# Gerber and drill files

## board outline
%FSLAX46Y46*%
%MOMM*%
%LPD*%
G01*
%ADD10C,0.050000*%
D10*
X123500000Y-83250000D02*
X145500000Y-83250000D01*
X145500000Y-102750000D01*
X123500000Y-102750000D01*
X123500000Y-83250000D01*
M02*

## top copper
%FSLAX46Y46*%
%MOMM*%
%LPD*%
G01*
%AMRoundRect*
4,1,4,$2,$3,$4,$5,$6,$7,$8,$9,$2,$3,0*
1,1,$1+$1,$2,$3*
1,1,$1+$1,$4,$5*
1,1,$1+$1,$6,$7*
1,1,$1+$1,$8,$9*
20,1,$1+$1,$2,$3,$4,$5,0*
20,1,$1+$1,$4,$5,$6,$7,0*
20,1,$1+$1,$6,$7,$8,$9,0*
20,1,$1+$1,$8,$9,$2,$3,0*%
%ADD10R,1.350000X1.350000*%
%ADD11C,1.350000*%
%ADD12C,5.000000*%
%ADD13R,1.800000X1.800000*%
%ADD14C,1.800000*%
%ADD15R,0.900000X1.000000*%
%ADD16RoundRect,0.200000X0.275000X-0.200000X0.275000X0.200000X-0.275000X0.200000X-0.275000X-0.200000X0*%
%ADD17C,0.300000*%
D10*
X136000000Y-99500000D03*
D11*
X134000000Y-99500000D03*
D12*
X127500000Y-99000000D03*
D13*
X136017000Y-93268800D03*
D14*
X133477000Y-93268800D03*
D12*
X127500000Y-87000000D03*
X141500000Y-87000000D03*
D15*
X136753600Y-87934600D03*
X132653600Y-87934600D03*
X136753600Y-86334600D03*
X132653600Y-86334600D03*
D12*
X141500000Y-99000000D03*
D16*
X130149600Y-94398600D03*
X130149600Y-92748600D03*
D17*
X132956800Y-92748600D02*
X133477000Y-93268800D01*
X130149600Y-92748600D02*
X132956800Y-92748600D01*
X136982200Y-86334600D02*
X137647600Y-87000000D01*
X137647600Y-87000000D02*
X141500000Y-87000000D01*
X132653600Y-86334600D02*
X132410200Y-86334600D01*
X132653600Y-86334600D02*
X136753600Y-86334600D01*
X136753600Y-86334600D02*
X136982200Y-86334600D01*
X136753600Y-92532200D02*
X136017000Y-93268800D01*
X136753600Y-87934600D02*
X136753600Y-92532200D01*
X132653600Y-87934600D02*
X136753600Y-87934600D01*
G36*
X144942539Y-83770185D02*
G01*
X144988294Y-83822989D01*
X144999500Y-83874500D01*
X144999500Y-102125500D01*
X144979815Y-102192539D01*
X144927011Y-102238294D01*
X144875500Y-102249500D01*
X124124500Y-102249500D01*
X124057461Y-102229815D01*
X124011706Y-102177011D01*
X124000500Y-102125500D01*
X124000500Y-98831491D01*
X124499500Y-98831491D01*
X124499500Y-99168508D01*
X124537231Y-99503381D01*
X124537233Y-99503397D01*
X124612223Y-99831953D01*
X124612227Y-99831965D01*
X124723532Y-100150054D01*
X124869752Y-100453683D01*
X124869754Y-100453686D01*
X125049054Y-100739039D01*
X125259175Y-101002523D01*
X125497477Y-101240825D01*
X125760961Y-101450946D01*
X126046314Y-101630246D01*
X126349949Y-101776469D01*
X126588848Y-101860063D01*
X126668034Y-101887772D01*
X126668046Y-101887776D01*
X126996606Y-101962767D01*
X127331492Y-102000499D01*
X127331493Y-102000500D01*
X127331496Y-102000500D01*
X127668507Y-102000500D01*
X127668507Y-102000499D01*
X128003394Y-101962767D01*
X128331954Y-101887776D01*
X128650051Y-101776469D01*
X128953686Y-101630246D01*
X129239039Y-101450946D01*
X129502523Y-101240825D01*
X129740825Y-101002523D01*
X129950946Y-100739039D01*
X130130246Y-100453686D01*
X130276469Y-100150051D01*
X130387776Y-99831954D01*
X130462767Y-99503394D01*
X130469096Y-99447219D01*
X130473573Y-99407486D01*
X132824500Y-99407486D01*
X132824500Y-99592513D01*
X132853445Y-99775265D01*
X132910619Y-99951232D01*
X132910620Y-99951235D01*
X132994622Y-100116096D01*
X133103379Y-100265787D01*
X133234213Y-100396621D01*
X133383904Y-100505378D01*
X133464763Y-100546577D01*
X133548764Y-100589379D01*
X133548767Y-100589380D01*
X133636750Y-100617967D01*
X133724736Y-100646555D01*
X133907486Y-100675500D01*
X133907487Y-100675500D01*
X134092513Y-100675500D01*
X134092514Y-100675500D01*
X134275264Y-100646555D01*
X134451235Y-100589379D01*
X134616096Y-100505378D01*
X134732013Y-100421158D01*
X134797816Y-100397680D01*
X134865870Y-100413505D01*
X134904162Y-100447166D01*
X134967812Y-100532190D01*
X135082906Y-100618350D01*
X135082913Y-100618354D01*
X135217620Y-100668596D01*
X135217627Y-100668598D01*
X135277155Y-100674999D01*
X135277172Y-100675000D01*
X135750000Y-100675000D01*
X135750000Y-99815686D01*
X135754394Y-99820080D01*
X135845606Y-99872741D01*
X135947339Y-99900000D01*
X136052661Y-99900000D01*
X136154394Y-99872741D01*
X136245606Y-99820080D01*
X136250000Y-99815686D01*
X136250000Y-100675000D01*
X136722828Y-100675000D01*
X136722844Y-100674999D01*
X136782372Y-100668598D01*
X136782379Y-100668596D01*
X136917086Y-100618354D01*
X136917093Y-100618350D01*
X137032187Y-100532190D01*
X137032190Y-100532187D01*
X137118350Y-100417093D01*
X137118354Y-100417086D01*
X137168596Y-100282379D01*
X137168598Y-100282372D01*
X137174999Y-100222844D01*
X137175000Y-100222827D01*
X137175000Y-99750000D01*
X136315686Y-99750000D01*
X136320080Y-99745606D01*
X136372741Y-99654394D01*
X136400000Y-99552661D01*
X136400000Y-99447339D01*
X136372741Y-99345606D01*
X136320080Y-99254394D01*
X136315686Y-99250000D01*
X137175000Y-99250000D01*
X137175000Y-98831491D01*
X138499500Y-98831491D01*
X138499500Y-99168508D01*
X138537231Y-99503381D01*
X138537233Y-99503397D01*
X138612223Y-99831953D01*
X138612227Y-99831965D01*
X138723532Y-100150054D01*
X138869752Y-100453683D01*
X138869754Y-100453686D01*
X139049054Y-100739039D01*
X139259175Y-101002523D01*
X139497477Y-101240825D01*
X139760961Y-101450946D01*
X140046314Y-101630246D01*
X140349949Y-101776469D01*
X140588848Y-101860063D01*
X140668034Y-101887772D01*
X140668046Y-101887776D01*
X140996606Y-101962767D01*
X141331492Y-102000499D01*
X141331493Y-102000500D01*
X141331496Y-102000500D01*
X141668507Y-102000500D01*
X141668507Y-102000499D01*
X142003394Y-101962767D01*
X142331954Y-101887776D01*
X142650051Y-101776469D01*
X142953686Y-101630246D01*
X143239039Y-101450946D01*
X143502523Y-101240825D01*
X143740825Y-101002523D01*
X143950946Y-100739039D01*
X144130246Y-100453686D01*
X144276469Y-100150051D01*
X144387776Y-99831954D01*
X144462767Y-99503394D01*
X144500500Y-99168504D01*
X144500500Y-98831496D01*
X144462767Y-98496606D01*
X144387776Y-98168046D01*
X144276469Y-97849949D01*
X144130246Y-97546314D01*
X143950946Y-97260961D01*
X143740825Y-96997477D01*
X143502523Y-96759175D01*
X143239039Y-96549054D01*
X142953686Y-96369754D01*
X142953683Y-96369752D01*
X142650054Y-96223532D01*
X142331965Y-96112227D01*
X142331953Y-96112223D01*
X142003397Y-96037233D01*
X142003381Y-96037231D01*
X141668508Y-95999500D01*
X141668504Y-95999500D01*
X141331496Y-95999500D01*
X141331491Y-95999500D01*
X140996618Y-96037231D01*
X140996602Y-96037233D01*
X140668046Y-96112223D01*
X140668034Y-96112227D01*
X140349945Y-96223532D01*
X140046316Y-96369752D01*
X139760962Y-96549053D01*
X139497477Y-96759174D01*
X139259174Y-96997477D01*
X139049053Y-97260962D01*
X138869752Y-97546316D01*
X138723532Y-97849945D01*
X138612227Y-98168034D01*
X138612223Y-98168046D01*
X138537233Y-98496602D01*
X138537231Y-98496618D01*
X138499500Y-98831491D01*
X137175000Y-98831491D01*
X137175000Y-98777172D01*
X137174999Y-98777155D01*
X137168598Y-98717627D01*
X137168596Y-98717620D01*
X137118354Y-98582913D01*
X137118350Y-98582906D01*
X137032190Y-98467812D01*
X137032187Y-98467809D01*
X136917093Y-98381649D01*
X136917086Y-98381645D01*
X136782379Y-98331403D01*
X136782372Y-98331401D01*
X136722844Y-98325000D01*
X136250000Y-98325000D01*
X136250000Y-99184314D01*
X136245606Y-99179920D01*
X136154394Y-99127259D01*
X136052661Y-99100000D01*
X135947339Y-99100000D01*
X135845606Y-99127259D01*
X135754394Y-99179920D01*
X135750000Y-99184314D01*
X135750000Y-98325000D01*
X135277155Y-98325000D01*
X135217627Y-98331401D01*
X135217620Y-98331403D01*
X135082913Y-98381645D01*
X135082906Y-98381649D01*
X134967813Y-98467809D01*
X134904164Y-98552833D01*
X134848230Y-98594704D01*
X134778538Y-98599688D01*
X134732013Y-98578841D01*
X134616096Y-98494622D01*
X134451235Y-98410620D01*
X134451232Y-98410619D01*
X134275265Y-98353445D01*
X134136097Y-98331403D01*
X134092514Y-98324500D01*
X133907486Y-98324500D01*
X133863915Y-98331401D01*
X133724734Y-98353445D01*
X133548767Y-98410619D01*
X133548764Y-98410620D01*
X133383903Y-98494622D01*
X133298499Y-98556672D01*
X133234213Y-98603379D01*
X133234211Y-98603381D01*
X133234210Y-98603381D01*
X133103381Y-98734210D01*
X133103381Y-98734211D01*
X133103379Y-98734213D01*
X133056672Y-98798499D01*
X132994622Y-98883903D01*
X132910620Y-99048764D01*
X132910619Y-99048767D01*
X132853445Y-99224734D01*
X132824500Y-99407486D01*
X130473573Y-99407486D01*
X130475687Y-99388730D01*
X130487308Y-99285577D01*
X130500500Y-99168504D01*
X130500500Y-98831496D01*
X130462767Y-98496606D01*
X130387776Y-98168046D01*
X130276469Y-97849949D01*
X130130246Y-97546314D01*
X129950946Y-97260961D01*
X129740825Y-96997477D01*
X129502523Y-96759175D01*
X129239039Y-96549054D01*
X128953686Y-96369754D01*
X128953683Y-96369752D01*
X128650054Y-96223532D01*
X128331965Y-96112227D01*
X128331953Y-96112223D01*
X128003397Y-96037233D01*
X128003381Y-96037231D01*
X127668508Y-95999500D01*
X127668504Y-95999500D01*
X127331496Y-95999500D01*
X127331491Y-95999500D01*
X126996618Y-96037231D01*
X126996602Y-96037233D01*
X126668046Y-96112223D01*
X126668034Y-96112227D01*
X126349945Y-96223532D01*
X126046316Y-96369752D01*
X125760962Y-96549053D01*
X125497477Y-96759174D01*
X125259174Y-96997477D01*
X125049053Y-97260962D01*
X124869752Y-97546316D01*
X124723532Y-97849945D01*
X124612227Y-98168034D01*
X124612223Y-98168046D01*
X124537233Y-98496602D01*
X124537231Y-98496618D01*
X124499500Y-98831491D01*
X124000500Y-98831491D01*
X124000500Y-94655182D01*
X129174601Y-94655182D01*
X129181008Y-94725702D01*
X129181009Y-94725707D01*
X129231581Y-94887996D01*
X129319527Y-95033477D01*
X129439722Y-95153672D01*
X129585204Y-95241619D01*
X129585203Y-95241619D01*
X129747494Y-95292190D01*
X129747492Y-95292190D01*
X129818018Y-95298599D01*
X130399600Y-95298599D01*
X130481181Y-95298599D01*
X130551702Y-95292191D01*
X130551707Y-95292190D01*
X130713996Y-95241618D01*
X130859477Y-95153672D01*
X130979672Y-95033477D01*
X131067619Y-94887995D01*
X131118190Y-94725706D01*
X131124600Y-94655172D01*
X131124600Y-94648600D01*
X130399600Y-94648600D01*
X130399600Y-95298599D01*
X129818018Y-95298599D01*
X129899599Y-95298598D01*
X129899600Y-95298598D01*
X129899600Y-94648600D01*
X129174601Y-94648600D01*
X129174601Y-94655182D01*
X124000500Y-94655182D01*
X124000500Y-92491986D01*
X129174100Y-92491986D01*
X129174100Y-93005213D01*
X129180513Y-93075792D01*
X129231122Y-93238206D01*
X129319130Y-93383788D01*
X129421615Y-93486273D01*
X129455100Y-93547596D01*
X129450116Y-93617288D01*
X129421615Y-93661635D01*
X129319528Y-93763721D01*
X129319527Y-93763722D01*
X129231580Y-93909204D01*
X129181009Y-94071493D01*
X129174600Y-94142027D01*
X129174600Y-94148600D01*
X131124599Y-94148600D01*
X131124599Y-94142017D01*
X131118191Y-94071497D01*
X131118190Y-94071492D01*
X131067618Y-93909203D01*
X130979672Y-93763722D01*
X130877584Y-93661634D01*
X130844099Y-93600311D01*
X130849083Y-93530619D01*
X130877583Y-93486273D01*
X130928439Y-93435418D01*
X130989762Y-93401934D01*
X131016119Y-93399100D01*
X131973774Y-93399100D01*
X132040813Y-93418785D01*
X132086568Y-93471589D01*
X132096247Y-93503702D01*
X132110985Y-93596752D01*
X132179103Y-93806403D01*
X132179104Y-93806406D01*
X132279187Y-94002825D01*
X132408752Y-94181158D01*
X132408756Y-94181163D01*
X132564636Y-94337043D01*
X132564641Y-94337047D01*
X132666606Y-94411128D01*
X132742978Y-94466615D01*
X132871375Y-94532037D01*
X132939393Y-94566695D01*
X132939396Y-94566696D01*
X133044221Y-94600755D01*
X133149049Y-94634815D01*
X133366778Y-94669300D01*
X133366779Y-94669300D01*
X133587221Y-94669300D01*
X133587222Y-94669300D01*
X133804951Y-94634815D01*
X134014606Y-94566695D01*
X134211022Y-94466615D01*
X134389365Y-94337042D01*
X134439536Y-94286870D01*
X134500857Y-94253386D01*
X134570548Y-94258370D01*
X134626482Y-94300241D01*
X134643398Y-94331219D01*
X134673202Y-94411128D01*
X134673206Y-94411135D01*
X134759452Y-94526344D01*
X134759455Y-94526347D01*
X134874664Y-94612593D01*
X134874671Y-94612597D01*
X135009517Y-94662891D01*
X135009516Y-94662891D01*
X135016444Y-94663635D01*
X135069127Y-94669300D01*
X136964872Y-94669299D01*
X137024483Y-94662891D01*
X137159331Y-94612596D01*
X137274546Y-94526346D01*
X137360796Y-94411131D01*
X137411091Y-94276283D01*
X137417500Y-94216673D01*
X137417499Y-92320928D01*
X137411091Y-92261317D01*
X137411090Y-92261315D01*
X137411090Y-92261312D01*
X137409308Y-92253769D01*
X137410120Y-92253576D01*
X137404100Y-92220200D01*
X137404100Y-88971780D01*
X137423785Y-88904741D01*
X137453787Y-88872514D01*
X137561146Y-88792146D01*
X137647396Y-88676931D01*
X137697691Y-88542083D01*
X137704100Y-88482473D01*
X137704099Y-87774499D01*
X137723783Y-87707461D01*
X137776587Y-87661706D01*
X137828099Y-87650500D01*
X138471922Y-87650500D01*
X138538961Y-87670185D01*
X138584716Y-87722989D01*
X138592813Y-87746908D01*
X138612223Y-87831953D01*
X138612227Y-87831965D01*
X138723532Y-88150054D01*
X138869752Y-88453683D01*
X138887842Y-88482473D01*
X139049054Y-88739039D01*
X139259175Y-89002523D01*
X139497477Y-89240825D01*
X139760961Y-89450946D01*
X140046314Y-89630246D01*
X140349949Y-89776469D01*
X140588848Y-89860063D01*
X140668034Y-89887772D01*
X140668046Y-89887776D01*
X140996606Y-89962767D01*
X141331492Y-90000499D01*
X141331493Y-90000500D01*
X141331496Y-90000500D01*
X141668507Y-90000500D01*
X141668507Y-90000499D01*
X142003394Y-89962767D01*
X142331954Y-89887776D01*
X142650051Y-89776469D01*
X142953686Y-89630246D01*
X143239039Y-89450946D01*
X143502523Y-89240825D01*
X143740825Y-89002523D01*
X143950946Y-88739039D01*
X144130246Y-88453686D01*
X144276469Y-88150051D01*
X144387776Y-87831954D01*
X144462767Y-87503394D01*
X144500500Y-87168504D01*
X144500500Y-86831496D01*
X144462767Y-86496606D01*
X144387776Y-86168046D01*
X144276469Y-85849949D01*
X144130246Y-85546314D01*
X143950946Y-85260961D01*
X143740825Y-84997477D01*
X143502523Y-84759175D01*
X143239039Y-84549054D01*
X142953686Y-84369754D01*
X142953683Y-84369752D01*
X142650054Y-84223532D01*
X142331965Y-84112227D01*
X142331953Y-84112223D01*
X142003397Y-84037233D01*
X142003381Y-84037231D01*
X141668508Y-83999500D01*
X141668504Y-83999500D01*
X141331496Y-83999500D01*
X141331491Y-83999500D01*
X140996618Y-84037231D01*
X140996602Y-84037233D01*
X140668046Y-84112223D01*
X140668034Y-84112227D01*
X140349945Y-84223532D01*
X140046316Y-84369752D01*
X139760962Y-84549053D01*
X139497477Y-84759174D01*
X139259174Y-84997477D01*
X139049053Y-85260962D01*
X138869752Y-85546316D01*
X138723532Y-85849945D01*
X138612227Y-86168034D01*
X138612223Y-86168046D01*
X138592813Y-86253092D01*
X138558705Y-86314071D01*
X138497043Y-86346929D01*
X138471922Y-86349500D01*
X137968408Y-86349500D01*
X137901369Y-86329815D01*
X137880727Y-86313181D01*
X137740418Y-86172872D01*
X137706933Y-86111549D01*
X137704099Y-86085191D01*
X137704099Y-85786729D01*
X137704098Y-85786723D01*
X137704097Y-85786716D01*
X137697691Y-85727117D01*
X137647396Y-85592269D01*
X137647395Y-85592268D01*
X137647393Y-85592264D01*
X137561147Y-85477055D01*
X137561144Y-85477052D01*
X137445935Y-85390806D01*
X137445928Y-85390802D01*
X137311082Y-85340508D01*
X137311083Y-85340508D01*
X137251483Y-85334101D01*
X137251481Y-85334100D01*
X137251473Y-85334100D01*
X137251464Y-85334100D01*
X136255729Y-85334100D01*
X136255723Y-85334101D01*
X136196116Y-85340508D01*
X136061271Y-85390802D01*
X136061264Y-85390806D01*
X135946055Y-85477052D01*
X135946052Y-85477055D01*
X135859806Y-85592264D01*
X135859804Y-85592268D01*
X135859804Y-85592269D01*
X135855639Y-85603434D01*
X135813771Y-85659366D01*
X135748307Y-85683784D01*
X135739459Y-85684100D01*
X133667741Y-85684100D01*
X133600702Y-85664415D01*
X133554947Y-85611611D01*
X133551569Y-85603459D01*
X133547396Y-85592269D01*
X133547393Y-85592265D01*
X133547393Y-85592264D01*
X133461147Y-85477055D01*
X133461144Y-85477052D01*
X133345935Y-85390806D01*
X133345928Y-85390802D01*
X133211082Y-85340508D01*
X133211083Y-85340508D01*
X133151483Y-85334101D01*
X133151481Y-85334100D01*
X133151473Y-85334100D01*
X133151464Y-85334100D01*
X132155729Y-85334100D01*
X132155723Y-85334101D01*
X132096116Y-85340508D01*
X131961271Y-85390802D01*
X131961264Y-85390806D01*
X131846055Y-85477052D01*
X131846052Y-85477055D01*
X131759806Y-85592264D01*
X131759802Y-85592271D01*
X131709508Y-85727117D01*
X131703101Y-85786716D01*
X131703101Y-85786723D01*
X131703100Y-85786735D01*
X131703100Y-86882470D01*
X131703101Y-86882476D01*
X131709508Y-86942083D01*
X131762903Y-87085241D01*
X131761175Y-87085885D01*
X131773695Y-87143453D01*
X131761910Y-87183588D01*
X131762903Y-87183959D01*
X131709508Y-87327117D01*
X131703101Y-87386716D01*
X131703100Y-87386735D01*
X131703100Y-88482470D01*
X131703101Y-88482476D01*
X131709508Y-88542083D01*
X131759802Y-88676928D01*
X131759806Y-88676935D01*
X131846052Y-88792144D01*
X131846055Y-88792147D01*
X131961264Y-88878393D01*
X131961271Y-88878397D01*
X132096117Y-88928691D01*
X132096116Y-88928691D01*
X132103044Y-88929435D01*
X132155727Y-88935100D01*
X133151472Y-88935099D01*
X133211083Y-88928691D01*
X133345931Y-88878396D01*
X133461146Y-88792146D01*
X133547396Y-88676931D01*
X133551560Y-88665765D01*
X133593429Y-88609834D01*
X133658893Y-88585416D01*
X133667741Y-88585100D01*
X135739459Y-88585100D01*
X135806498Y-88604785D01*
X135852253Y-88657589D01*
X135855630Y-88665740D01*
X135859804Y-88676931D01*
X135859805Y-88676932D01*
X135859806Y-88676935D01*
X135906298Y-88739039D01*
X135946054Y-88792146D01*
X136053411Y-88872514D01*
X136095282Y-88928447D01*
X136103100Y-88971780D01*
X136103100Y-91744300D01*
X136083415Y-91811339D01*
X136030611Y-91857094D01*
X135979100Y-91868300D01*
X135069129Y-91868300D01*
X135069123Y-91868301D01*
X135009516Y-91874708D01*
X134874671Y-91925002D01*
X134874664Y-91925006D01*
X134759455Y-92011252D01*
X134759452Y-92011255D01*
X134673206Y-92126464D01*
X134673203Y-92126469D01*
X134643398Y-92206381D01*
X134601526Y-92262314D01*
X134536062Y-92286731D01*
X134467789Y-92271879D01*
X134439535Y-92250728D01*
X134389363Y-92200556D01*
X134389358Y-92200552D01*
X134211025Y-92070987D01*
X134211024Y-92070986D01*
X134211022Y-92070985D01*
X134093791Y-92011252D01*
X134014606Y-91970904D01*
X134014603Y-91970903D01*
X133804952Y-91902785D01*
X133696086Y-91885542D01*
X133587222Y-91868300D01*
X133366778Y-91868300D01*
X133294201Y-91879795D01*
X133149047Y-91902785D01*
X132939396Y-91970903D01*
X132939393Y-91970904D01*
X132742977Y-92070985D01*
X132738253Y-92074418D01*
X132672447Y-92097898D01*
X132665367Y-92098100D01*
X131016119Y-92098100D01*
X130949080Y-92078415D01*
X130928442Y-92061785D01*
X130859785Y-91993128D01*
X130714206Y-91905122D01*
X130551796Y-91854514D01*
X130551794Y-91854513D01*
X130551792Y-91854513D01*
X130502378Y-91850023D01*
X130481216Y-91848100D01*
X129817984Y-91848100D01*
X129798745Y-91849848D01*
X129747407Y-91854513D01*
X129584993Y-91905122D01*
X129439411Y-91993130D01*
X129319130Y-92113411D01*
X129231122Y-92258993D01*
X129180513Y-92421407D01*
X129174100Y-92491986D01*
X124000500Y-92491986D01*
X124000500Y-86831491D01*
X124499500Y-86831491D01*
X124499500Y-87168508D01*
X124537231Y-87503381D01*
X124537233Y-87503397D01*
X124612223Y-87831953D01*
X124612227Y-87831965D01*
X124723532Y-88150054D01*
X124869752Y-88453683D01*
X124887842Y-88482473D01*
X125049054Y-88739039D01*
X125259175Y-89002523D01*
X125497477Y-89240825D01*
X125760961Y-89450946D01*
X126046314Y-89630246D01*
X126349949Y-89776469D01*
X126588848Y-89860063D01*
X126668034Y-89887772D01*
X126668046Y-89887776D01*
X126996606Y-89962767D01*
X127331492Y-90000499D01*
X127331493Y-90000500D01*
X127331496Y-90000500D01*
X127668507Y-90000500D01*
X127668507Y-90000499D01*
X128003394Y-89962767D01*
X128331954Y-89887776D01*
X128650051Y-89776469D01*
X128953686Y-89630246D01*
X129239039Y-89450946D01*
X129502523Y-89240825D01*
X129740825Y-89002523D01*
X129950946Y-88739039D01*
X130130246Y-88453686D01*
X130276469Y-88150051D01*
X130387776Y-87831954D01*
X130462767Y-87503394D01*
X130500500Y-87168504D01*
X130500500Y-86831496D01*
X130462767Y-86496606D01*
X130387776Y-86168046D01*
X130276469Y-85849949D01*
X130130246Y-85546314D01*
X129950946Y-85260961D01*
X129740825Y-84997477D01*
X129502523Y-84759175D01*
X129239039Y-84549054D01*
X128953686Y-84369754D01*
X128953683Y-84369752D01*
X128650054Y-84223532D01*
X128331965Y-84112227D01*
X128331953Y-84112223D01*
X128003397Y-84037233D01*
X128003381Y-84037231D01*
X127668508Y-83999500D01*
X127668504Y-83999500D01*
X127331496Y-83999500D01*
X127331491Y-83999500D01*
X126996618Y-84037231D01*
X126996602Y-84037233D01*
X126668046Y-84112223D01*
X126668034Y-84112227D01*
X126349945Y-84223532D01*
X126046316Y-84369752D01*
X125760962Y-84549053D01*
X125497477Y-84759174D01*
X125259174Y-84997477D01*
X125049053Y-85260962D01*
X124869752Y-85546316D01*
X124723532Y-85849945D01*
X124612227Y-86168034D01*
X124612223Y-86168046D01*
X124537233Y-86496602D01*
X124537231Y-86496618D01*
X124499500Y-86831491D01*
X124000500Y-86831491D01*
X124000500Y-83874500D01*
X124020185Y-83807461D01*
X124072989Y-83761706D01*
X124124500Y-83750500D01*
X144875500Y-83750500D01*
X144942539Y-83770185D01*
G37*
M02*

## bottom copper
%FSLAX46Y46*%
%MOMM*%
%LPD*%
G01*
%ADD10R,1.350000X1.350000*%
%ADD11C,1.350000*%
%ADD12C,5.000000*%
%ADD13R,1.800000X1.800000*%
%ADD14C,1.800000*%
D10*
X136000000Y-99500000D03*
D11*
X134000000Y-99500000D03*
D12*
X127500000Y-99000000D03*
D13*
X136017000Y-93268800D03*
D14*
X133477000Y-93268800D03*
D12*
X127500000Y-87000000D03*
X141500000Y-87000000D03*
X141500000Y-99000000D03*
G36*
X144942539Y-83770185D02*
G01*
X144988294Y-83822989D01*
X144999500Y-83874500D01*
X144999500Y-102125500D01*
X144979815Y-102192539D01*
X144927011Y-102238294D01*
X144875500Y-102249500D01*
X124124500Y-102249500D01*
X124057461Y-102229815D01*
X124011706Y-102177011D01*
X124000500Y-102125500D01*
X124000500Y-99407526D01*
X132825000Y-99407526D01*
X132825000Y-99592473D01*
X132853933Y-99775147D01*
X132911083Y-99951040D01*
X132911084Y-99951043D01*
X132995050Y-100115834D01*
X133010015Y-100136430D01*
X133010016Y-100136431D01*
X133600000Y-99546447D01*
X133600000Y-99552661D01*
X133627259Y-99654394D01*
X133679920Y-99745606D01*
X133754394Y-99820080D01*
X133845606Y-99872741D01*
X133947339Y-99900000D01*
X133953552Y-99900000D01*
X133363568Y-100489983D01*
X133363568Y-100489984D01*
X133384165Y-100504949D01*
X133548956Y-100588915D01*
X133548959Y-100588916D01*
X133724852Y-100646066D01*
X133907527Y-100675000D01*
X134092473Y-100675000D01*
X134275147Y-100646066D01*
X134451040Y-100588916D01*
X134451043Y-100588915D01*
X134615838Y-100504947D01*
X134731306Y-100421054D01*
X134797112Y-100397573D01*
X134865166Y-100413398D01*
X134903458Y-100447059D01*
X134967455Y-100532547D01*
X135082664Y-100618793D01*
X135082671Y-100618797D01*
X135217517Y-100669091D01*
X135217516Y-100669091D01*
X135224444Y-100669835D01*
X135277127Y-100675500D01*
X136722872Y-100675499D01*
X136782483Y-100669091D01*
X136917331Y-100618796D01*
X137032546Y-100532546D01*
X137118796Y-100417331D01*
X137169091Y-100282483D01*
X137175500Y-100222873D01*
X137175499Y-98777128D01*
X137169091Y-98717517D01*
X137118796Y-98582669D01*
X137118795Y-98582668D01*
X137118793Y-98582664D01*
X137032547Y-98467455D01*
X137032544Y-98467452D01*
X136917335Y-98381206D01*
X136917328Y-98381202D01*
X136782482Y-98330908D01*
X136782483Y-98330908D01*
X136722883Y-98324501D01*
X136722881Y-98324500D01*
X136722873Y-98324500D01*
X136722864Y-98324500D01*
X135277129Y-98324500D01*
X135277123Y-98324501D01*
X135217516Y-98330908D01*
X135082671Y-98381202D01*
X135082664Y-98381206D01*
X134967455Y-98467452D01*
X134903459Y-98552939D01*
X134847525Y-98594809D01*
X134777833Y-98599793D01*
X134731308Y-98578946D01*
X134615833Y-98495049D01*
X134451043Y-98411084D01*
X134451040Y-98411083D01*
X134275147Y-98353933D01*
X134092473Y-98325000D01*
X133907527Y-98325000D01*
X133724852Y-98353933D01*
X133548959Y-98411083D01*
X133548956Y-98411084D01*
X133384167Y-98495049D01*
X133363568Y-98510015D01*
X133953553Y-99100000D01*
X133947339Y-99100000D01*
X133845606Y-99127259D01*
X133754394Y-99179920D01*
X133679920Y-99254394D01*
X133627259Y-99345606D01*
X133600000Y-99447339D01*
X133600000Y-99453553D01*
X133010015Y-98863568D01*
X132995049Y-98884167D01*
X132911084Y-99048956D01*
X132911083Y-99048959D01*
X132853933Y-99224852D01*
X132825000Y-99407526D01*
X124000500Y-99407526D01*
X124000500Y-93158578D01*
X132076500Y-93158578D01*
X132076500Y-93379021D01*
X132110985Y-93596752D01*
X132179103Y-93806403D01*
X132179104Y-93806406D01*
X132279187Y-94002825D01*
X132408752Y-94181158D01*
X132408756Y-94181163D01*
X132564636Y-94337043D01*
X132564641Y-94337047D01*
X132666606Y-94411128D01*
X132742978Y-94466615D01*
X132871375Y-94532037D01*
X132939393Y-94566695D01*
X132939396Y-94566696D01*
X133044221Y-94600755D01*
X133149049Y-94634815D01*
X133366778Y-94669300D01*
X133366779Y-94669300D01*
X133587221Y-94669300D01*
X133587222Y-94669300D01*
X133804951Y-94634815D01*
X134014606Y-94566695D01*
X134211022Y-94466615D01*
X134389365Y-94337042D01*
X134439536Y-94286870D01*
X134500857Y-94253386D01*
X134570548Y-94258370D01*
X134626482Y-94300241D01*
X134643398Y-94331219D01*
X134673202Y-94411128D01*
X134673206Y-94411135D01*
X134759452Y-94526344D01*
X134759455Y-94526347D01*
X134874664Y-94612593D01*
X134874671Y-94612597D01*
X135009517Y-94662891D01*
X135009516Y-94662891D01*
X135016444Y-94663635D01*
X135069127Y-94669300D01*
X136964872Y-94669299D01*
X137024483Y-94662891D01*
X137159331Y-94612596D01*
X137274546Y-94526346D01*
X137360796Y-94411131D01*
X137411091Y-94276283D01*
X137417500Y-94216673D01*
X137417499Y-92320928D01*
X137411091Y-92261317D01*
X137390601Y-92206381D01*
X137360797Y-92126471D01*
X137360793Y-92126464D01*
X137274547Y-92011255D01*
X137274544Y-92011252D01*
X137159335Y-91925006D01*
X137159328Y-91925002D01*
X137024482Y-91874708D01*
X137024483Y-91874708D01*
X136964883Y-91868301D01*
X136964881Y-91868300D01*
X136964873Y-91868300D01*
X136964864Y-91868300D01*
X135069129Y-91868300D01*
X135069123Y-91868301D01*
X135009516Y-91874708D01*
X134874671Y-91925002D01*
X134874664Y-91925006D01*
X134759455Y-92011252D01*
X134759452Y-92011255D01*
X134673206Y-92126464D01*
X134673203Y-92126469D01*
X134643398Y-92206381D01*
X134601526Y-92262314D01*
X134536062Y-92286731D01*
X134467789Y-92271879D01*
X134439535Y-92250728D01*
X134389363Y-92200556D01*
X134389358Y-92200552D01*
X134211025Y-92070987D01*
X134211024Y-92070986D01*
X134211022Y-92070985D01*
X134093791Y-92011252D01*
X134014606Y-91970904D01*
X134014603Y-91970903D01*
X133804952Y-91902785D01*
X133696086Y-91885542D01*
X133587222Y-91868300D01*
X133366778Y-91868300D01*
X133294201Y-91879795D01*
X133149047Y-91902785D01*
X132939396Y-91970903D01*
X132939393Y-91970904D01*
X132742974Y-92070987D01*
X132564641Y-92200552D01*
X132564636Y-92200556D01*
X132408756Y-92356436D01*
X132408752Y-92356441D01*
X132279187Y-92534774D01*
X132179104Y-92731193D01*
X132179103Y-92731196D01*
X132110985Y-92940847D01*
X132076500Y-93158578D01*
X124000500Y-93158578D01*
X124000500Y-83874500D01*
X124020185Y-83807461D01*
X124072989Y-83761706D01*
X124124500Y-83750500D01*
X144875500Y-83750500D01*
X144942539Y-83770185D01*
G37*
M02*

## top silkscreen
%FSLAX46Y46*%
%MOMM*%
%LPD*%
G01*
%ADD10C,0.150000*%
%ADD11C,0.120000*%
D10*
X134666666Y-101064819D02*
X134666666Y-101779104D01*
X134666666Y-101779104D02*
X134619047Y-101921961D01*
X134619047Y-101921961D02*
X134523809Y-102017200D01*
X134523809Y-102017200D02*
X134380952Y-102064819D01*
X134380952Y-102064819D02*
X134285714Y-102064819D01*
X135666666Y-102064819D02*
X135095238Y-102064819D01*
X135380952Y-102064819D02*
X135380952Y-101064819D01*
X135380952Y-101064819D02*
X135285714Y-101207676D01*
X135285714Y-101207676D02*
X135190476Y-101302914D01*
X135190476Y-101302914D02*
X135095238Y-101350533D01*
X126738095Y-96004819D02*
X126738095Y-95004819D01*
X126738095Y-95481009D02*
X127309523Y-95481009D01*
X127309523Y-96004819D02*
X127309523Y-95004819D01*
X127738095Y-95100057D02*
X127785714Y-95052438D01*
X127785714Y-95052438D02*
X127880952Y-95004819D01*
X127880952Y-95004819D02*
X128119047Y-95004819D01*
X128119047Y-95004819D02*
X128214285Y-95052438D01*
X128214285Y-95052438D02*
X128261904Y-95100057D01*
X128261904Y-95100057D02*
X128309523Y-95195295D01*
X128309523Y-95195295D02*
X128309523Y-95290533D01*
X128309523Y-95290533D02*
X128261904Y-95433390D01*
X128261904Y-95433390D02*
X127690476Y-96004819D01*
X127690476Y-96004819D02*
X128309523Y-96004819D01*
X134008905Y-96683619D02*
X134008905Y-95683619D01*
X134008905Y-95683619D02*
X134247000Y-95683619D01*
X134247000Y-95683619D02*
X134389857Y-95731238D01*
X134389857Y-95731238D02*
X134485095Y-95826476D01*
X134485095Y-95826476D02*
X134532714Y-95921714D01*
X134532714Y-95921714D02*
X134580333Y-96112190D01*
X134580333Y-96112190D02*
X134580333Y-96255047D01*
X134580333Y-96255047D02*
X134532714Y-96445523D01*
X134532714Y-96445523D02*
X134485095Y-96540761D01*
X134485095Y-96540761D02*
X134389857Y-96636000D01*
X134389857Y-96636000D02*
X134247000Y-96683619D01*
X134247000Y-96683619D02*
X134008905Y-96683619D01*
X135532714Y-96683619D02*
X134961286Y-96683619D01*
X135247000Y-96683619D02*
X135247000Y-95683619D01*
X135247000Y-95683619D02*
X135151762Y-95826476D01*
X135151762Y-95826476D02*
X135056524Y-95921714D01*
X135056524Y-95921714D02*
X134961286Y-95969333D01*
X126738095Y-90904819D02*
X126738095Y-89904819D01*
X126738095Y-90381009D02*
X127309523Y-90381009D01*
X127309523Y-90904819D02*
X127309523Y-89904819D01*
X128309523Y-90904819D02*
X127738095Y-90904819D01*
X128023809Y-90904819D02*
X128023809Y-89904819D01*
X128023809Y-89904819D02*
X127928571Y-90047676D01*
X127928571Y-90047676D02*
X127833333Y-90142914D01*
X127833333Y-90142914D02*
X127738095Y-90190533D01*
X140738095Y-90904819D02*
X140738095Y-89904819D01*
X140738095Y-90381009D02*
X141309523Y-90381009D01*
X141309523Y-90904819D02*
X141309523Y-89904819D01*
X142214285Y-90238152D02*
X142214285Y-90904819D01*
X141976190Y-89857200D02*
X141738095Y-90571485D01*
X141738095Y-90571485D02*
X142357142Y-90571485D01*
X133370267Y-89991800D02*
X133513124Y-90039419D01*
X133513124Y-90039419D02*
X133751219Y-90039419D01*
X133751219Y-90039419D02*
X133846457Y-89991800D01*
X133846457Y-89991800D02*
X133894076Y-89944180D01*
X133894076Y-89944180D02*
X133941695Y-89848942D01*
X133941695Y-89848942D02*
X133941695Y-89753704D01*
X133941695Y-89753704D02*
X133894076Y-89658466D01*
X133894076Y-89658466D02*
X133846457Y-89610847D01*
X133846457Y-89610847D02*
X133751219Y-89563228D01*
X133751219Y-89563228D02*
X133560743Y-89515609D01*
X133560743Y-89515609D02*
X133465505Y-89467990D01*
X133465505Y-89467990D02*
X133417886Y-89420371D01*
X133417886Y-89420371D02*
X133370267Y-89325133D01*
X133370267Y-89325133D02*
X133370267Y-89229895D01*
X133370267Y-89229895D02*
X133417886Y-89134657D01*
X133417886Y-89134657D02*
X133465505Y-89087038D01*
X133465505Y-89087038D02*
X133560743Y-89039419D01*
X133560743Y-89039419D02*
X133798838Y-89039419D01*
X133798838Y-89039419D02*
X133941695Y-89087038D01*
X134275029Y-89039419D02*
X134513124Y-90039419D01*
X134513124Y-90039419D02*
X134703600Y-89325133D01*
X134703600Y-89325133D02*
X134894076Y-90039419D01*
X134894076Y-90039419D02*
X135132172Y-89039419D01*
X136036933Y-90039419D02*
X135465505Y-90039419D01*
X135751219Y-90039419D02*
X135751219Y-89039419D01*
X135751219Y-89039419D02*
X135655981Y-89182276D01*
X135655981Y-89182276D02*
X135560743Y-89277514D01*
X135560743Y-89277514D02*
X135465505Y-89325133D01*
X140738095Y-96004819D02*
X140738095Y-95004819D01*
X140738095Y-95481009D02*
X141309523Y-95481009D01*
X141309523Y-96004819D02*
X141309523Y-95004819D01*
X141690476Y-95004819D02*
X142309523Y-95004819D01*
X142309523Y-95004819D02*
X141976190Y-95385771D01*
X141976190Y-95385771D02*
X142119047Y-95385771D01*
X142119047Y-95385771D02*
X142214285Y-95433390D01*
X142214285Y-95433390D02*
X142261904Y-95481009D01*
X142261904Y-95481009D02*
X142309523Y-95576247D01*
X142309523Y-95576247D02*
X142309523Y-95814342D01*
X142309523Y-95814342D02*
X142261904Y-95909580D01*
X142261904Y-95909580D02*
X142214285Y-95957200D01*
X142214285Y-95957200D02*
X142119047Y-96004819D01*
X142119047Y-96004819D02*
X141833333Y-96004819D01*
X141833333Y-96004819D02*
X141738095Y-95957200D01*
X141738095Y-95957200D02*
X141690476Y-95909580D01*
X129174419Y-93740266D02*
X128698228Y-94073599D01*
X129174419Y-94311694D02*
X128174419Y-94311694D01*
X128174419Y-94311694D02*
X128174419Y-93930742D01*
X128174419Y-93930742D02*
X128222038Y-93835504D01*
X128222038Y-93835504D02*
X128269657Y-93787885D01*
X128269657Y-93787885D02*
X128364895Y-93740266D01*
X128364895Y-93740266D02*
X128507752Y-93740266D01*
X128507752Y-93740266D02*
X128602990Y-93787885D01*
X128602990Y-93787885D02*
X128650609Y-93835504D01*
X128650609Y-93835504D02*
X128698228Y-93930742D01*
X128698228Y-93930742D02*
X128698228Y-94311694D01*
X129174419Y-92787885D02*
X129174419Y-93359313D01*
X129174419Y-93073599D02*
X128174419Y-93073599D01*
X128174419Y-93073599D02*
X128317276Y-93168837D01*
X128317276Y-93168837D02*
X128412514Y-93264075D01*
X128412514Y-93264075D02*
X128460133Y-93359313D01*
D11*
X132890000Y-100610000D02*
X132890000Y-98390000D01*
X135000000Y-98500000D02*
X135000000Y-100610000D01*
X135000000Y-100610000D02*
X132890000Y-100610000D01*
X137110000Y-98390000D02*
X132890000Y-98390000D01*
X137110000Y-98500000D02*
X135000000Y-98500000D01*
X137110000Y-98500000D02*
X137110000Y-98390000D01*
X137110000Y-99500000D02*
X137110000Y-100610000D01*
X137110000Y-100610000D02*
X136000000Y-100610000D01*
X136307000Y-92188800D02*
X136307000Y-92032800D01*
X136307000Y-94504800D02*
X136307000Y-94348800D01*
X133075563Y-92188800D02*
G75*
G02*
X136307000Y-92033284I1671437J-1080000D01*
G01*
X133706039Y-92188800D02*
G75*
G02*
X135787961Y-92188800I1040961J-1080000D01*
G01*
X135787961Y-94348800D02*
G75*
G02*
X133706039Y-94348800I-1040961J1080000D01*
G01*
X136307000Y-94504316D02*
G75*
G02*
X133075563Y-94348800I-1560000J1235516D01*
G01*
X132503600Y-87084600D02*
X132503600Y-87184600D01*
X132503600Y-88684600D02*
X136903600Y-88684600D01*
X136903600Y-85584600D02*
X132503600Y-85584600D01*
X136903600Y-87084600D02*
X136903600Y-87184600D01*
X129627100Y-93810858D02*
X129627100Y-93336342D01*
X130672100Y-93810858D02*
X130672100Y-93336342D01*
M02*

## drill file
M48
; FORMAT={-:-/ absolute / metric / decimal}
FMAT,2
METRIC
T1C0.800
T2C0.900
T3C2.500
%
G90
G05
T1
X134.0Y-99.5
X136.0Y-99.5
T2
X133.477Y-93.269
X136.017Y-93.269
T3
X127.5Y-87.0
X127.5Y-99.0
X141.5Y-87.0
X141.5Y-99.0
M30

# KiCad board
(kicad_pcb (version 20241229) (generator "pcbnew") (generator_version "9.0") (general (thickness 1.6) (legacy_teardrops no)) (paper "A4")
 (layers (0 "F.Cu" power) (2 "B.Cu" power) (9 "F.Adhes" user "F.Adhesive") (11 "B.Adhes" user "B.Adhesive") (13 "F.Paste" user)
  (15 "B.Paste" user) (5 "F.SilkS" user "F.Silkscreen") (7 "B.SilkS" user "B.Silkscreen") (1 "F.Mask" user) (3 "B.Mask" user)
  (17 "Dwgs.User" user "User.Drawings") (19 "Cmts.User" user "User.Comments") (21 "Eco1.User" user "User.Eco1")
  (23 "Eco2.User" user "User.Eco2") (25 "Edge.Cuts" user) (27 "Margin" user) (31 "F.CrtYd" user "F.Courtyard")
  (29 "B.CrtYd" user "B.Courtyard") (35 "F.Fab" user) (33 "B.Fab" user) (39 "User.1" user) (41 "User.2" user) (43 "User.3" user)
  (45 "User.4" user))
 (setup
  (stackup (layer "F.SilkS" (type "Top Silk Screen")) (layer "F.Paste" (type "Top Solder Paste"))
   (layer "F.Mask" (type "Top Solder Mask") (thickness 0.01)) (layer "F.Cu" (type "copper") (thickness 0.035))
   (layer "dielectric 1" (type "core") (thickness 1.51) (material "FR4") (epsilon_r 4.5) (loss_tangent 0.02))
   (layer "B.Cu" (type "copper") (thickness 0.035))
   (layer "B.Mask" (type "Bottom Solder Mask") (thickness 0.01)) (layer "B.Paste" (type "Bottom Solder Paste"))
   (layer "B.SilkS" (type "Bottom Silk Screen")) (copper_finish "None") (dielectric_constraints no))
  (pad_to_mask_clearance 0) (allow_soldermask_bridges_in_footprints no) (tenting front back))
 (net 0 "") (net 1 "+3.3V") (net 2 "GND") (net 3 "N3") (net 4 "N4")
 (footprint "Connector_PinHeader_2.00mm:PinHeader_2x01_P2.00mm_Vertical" (layer "F.Cu") (at 136 99.5 180)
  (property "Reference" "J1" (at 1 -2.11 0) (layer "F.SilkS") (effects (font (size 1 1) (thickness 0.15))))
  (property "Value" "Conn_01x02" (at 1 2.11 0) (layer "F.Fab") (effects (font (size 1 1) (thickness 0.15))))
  (fp_line (start 3.11 -1.11) (end 3.11 1.11) (stroke (width 0.12) (type solid)) (layer "F.SilkS"))
  (fp_line (start 1 1) (end 1 -1.11) (stroke (width 0.12) (type solid)) (layer "F.SilkS"))
  (fp_line (start 1 -1.11) (end 3.11 -1.11) (stroke (width 0.12) (type solid)) (layer "F.SilkS"))
  (fp_line (start -1.11 1.11) (end 3.11 1.11) (stroke (width 0.12) (type solid)) (layer "F.SilkS"))
  (fp_line (start -1.11 1) (end 1 1) (stroke (width 0.12) (type solid)) (layer "F.SilkS"))
  (fp_line (start -1.11 1) (end -1.11 1.11) (stroke (width 0.12) (type solid)) (layer "F.SilkS"))
  (fp_line (start -1.11 0) (end -1.11 -1.11) (stroke (width 0.12) (type solid)) (layer "F.SilkS"))
  (fp_line (start -1.11 -1.11) (end 0 -1.11) (stroke (width 0.12) (type solid)) (layer "F.SilkS"))
  (pad "1" thru_hole rect (at 0 0 180) (size 1.35 1.35) (drill 0.8) (layers "*.Cu" "*.Mask") (remove_unused_layers no) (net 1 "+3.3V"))
  (pad "2" thru_hole circle (at 2 0 180) (size 1.35 1.35) (drill 0.8) (layers "*.Cu" "*.Mask") (remove_unused_layers no) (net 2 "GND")))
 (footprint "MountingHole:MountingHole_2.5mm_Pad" (layer "F.Cu") (at 127.5 99)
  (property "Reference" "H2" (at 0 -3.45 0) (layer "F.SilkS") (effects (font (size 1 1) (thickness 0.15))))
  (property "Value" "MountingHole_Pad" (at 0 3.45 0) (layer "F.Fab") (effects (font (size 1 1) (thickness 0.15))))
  (pad "1" thru_hole circle (at 0 0) (size 5 5) (drill 2.5) (layers "*.Cu" "*.Mask") (remove_unused_layers no) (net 2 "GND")
   (zone_connect 2)))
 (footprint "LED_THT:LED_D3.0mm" (layer "F.Cu") (at 136.017 93.2688 180)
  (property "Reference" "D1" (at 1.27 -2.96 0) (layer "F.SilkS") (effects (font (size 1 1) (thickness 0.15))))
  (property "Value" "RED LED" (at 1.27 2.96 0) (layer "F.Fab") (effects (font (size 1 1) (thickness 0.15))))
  (fp_line (start -0.29 1.08) (end -0.29 1.236) (stroke (width 0.12) (type solid)) (layer "F.SilkS"))
  (fp_line (start -0.29 -1.236) (end -0.29 -1.08) (stroke (width 0.12) (type solid)) (layer "F.SilkS"))
  (fp_arc (start 2.941437 1.08) (mid 1.36566 1.987699) (end -0.29 1.235516) (stroke (width 0.12) (type solid)) (layer "F.SilkS"))
  (fp_arc (start 2.310961 1.08) (mid 1.27 1.5) (end 0.229039 1.08) (stroke (width 0.12) (type solid)) (layer "F.SilkS"))
  (fp_arc (start 0.229039 -1.08) (mid 1.27 -1.5) (end 2.310961 -1.08) (stroke (width 0.12) (type solid)) (layer "F.SilkS"))
  (fp_arc (start -0.29 -1.235516) (mid 1.36566 -1.987699) (end 2.941437 -1.08) (stroke (width 0.12) (type solid)) (layer "F.SilkS"))
  (pad "1" thru_hole rect (at 0 0 180) (size 1.8 1.8) (drill 0.9) (layers "*.Cu" "*.Mask") (remove_unused_layers no) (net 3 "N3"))
  (pad "2" thru_hole circle (at 2.54 0 180) (size 1.8 1.8) (drill 0.9) (layers "*.Cu" "*.Mask") (remove_unused_layers no) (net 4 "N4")))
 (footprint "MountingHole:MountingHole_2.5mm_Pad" (layer "F.Cu") (at 127.5 87 180)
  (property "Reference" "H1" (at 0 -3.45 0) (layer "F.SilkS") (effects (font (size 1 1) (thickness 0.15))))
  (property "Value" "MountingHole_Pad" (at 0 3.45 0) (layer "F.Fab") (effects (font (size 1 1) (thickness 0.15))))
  (pad "1" thru_hole circle (at 0 0 180) (size 5 5) (drill 2.5) (layers "*.Cu" "*.Mask") (remove_unused_layers no) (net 2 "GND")
   (zone_connect 2)))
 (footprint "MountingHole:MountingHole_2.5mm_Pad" (layer "F.Cu") (at 141.5 87 180)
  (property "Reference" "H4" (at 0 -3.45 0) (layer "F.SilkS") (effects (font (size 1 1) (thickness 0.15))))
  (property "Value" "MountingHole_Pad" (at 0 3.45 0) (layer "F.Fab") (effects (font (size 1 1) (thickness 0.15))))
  (pad "1" thru_hole circle (at 0 0 180) (size 5 5) (drill 2.5) (layers "*.Cu" "*.Mask") (remove_unused_layers no) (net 2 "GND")
   (zone_connect 2)))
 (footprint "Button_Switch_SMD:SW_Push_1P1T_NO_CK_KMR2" (layer "F.Cu") (at 134.7036 87.1346 180)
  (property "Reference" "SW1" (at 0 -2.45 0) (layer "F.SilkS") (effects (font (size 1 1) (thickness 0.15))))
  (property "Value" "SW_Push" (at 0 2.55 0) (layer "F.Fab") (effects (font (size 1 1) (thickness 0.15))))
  (fp_line (start 2.2 0.05) (end 2.2 -0.05) (stroke (width 0.12) (type solid)) (layer "F.SilkS"))
  (fp_line (start 2.2 -1.55) (end -2.2 -1.55) (stroke (width 0.12) (type solid)) (layer "F.SilkS"))
  (fp_line (start -2.2 1.55) (end 2.2 1.55) (stroke (width 0.12) (type solid)) (layer "F.SilkS"))
  (fp_line (start -2.2 0.05) (end -2.2 -0.05) (stroke (width 0.12) (type solid)) (layer "F.SilkS"))
  (pad "1" smd rect (at -2.05 -0.8 180) (size 0.9 1) (layers "F.Cu" "F.Mask" "F.Paste") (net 3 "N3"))
  (pad "1" smd rect (at 2.05 -0.8 180) (size 0.9 1) (layers "F.Cu" "F.Mask" "F.Paste") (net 3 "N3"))
  (pad "2" smd rect (at -2.05 0.8 180) (size 0.9 1) (layers "F.Cu" "F.Mask" "F.Paste") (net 2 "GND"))
  (pad "2" smd rect (at 2.05 0.8 180) (size 0.9 1) (layers "F.Cu" "F.Mask" "F.Paste") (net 2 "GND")))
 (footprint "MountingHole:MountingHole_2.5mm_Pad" (layer "F.Cu") (at 141.5 99)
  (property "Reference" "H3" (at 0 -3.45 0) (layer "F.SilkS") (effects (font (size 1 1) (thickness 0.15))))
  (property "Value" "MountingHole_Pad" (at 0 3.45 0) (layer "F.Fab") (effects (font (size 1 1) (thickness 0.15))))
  (pad "1" thru_hole circle (at 0 0) (size 5 5) (drill 2.5) (layers "*.Cu" "*.Mask") (remove_unused_layers no) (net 2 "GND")
   (zone_connect 2)))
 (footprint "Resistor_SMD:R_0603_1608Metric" (layer "F.Cu") (at 130.1496 93.5736 90)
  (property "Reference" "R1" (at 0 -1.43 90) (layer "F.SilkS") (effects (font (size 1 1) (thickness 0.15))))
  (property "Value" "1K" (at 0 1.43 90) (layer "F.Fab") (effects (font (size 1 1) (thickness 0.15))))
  (fp_line (start -0.237258 -0.5225) (end 0.237258 -0.5225) (stroke (width 0.12) (type solid)) (layer "F.SilkS"))
  (fp_line (start -0.237258 0.5225) (end 0.237258 0.5225) (stroke (width 0.12) (type solid)) (layer "F.SilkS"))
  (pad "1" smd roundrect (at -0.825 0 90) (size 0.8 0.95) (layers "F.Cu" "F.Mask" "F.Paste") (roundrect_rratio 0.25) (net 1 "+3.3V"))
  (pad "2" smd roundrect (at 0.825 0 90) (size 0.8 0.95) (layers "F.Cu" "F.Mask" "F.Paste") (roundrect_rratio 0.25) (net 4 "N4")))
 (gr_rect (start 123.5 83.25) (end 145.5 102.75) (stroke (width 0.05) (type default)) (fill no) (layer "Edge.Cuts"))
 (segment (start 132.9568 92.7486) (end 133.477 93.2688) (width 0.3) (layer "F.Cu") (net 4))
 (segment (start 130.1496 92.7486) (end 132.9568 92.7486) (width 0.3) (layer "F.Cu") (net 4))
 (segment (start 136.9822 86.3346) (end 137.6476 87) (width 0.3) (layer "F.Cu") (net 2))
 (segment (start 137.6476 87) (end 141.5 87) (width 0.3) (layer "F.Cu") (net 2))
 (segment (start 132.6536 86.3346) (end 132.4102 86.3346) (width 0.3) (layer "F.Cu") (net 2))
 (segment (start 132.6536 86.3346) (end 136.7536 86.3346) (width 0.3) (layer "F.Cu") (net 2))
 (segment (start 136.7536 86.3346) (end 136.9822 86.3346) (width 0.3) (layer "F.Cu") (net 2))
 (segment (start 136.7536 92.5322) (end 136.017 93.2688) (width 0.3) (layer "F.Cu") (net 3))
 (segment (start 136.7536 87.9346) (end 136.7536 92.5322) (width 0.3) (layer "F.Cu") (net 3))
 (segment (start 132.6536 87.9346) (end 136.7536 87.9346) (width 0.3) (layer "F.Cu") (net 3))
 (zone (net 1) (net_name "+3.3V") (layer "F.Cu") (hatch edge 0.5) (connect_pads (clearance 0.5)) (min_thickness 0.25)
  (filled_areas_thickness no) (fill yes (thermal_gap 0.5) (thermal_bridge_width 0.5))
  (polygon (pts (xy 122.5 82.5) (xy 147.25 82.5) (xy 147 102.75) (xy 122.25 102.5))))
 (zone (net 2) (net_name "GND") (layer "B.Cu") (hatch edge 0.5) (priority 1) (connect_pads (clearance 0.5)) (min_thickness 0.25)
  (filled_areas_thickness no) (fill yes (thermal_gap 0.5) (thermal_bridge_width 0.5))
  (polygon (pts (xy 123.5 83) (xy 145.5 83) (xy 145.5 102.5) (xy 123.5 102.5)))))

